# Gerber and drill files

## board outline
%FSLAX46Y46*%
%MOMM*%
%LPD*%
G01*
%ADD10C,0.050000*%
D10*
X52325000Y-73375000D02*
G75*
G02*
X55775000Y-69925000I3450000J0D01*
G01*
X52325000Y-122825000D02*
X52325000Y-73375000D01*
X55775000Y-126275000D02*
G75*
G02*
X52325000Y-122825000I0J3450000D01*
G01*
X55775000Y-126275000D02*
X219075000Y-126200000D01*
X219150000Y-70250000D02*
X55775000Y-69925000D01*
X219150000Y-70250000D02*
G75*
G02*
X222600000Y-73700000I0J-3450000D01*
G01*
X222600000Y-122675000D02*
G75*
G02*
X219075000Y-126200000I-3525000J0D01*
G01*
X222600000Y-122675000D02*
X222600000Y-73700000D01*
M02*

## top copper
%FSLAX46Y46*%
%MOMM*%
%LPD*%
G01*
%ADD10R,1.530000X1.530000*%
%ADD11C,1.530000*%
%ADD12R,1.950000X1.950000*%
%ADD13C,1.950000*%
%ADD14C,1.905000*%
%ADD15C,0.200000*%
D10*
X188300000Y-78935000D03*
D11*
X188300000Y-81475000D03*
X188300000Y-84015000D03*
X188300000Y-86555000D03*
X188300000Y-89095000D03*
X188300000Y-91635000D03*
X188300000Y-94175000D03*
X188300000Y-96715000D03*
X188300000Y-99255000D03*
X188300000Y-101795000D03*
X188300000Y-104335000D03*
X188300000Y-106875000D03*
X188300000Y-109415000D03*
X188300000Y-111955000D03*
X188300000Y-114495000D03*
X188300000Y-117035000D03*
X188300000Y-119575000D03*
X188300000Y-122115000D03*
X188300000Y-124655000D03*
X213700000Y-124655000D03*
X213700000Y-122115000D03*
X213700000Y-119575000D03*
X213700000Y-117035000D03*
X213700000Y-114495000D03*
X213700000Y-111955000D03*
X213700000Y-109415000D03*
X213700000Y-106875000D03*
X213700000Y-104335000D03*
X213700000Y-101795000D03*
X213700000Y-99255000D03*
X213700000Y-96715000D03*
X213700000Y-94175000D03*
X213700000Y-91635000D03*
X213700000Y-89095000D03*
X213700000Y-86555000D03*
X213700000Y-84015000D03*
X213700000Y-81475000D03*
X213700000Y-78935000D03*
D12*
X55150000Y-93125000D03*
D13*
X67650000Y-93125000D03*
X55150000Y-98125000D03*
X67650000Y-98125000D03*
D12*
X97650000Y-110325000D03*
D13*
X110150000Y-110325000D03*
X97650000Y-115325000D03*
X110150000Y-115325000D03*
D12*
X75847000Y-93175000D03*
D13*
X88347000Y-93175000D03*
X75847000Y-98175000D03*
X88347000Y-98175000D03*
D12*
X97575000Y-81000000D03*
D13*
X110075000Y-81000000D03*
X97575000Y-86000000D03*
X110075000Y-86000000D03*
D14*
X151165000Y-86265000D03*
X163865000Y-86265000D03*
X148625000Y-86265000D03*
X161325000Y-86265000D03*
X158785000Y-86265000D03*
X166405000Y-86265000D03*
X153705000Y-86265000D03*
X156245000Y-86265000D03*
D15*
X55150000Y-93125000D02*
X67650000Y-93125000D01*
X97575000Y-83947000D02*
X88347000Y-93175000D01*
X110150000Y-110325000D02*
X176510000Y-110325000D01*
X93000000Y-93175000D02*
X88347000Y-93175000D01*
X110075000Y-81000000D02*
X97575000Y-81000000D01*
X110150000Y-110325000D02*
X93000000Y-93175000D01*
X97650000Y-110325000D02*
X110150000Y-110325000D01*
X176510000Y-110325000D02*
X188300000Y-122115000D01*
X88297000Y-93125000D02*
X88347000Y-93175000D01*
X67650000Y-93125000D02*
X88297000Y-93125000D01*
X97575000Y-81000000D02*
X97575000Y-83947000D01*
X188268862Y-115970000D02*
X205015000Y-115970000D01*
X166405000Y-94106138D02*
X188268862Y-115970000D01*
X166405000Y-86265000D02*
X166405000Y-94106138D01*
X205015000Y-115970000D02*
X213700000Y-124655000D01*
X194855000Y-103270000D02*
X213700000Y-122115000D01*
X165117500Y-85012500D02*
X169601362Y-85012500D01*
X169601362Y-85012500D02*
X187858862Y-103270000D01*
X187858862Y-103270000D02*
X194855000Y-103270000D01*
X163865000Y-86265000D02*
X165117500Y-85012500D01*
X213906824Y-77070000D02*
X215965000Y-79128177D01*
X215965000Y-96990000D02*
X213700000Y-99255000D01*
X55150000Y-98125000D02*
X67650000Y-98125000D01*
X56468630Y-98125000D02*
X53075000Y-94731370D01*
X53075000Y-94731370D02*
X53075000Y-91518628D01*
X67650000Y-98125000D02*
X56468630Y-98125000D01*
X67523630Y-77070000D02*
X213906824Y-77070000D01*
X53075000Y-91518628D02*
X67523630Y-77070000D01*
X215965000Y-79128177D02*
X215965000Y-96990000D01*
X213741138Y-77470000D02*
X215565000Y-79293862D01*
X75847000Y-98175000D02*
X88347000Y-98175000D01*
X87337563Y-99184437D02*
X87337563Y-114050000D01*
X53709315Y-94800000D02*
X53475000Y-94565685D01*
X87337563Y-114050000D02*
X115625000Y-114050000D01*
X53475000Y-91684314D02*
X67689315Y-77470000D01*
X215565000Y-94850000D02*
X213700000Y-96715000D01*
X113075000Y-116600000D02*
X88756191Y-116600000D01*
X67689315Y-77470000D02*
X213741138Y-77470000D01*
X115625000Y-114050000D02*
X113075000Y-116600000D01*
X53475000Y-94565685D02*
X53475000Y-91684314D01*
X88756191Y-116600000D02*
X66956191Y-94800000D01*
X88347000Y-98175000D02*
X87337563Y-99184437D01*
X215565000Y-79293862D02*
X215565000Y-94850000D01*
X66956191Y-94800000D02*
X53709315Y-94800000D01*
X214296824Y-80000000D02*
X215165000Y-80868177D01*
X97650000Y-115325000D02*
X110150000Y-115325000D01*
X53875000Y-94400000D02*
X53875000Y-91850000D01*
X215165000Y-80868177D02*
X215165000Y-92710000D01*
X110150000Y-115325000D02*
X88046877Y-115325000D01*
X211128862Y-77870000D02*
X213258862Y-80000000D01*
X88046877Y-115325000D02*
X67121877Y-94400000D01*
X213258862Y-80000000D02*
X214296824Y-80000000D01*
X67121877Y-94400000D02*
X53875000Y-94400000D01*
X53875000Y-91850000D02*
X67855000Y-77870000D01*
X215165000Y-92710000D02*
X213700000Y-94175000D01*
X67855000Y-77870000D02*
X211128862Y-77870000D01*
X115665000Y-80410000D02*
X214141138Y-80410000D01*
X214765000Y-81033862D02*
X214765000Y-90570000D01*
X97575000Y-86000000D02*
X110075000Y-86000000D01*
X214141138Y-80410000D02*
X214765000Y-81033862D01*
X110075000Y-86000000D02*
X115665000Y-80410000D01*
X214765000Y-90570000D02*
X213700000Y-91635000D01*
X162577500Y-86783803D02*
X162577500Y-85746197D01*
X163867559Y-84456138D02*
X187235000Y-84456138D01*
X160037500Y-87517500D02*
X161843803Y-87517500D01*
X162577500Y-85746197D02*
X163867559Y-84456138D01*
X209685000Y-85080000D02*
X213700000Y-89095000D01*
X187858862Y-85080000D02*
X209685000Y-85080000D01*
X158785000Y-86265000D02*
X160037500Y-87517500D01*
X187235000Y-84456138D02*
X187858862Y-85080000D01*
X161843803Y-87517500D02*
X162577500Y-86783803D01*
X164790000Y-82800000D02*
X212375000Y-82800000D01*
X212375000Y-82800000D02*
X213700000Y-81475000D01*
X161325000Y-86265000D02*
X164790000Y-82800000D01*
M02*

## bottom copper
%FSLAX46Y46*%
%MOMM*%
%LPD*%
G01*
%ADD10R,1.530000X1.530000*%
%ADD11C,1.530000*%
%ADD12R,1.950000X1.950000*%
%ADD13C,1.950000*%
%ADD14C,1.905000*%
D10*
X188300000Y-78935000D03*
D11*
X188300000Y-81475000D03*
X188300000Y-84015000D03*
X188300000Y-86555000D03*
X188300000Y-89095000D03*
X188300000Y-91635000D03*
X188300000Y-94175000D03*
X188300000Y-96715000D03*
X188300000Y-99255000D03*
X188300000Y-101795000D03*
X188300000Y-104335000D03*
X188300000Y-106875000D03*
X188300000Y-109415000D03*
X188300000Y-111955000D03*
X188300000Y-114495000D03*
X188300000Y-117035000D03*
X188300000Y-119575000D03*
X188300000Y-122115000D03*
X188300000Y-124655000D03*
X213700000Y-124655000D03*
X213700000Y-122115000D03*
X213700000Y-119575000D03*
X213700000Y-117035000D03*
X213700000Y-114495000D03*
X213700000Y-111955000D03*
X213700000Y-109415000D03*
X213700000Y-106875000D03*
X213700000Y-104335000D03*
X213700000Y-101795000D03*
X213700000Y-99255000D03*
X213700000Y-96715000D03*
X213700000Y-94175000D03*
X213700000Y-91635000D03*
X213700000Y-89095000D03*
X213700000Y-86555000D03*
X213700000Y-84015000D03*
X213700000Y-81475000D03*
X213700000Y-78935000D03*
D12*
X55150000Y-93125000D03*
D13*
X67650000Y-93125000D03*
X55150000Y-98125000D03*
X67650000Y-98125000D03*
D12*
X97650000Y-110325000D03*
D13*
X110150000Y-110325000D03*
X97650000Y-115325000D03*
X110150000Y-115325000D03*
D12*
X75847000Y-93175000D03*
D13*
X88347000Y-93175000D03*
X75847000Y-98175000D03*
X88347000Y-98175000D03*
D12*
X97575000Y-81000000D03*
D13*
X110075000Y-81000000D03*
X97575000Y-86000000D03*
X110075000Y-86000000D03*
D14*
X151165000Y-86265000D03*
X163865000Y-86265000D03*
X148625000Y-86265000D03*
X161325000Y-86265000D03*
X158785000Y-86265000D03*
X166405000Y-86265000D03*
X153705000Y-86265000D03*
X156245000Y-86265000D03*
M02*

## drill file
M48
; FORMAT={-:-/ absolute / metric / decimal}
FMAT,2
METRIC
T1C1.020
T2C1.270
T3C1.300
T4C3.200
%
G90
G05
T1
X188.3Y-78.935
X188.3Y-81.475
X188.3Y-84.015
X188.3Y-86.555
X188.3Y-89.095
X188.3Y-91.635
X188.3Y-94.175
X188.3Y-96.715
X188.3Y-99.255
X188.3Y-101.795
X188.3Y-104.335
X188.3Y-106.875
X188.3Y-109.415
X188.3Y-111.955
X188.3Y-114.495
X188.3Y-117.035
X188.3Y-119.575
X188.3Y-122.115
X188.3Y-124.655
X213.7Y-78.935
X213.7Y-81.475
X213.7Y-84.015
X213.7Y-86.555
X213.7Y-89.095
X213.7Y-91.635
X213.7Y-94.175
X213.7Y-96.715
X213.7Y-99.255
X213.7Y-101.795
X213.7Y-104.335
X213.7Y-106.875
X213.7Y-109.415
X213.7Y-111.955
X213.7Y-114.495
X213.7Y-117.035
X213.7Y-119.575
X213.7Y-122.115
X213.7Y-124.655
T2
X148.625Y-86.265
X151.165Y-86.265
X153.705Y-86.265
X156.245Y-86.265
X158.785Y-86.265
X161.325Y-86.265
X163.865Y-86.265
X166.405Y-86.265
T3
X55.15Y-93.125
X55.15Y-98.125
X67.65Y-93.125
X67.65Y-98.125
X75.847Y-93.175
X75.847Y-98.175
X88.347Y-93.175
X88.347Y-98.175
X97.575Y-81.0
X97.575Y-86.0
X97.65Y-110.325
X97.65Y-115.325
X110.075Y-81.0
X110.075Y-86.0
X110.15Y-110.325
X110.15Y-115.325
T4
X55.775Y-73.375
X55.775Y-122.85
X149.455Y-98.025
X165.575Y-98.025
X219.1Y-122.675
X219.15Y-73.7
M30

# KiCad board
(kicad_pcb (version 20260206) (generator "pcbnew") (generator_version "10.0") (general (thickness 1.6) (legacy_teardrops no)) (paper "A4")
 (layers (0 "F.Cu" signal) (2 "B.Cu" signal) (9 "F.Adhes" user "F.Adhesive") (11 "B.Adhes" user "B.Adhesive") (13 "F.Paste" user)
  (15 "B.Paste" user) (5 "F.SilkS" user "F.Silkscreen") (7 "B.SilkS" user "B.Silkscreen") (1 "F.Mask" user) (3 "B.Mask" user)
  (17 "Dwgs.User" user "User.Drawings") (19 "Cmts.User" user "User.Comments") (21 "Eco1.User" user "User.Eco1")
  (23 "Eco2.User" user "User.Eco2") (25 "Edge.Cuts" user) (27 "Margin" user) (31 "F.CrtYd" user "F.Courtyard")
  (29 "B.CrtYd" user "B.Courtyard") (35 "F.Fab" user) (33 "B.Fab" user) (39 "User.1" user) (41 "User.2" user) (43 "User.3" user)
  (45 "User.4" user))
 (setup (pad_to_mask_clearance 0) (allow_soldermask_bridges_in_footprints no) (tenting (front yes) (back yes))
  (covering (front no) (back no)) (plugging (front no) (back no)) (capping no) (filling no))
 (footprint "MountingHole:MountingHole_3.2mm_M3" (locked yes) (layer "F.Cu") (at 55.775 122.85)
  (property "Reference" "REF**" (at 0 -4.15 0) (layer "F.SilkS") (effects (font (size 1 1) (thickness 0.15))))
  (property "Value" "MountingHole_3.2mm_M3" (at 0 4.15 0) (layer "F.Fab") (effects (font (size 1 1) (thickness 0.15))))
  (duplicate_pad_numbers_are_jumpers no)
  (pad "" np_thru_hole circle (at 0 0) (size 3.2 3.2) (drill 3.2) (layers "*.Cu" "*.Mask")))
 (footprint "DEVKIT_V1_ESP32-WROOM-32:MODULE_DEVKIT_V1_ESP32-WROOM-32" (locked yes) (layer "F.Cu") (at 201 101.785)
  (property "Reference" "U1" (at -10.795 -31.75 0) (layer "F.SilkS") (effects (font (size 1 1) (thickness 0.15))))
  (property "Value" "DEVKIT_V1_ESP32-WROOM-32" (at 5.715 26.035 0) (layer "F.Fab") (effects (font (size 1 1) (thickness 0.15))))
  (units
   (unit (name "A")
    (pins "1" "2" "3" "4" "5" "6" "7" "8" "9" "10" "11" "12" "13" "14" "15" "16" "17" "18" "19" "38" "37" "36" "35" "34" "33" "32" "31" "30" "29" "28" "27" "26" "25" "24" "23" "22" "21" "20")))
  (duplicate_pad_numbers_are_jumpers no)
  (pad "1" thru_hole rect (at -12.7 -22.85) (size 1.53 1.53) (drill 1.02) (layers "*.Cu" "*.Mask") (remove_unused_layers no)
   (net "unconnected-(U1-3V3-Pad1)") (solder_mask_margin 0.102))
  (pad "2" thru_hole circle (at -12.7 -20.31) (size 1.53 1.53) (drill 1.02) (layers "*.Cu" "*.Mask") (remove_unused_layers no)
   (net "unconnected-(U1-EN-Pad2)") (solder_mask_margin 0.102))
  (pad "3" thru_hole circle (at -12.7 -17.77) (size 1.53 1.53) (drill 1.02) (layers "*.Cu" "*.Mask") (remove_unused_layers no)
   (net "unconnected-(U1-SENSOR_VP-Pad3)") (solder_mask_margin 0.102))
  (pad "4" thru_hole circle (at -12.7 -15.23) (size 1.53 1.53) (drill 1.02) (layers "*.Cu" "*.Mask") (remove_unused_layers no)
   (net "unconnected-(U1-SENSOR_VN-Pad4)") (solder_mask_margin 0.102))
  (pad "5" thru_hole circle (at -12.7 -12.69) (size 1.53 1.53) (drill 1.02) (layers "*.Cu" "*.Mask") (remove_unused_layers no)
   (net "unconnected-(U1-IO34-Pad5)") (solder_mask_margin 0.102))
  (pad "6" thru_hole circle (at -12.7 -10.15) (size 1.53 1.53) (drill 1.02) (layers "*.Cu" "*.Mask") (remove_unused_layers no)
   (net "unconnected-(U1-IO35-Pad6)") (solder_mask_margin 0.102))
  (pad "7" thru_hole circle (at -12.7 -7.61) (size 1.53 1.53) (drill 1.02) (layers "*.Cu" "*.Mask") (remove_unused_layers no)
   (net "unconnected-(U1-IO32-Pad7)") (solder_mask_margin 0.102))
  (pad "8" thru_hole circle (at -12.7 -5.07) (size 1.53 1.53) (drill 1.02) (layers "*.Cu" "*.Mask") (remove_unused_layers no)
   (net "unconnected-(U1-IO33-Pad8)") (solder_mask_margin 0.102))
  (pad "9" thru_hole circle (at -12.7 -2.53) (size 1.53 1.53) (drill 1.02) (layers "*.Cu" "*.Mask") (remove_unused_layers no)
   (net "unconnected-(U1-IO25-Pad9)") (solder_mask_margin 0.102))
  (pad "10" thru_hole circle (at -12.7 0.01) (size 1.53 1.53) (drill 1.02) (layers "*.Cu" "*.Mask") (remove_unused_layers no)
   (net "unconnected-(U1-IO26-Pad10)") (solder_mask_margin 0.102))
  (pad "11" thru_hole circle (at -12.7 2.55) (size 1.53 1.53) (drill 1.02) (layers "*.Cu" "*.Mask") (remove_unused_layers no)
   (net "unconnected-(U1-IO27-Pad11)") (solder_mask_margin 0.102))
  (pad "12" thru_hole circle (at -12.7 5.09) (size 1.53 1.53) (drill 1.02) (layers "*.Cu" "*.Mask") (remove_unused_layers no)
   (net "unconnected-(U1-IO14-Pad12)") (solder_mask_margin 0.102))
  (pad "13" thru_hole circle (at -12.7 7.63) (size 1.53 1.53) (drill 1.02) (layers "*.Cu" "*.Mask") (remove_unused_layers no)
   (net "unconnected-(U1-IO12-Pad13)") (solder_mask_margin 0.102))
  (pad "14" thru_hole circle (at -12.7 10.17) (size 1.53 1.53) (drill 1.02) (layers "*.Cu" "*.Mask") (remove_unused_layers no)
   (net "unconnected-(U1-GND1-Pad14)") (solder_mask_margin 0.102))
  (pad "15" thru_hole circle (at -12.7 12.71) (size 1.53 1.53) (drill 1.02) (layers "*.Cu" "*.Mask") (remove_unused_layers no)
   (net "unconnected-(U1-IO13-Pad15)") (solder_mask_margin 0.102))
  (pad "16" thru_hole circle (at -12.7 15.25) (size 1.53 1.53) (drill 1.02) (layers "*.Cu" "*.Mask") (remove_unused_layers no)
   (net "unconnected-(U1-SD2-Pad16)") (solder_mask_margin 0.102))
  (pad "17" thru_hole circle (at -12.7 17.79) (size 1.53 1.53) (drill 1.02) (layers "*.Cu" "*.Mask") (remove_unused_layers no)
   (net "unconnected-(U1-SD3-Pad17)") (solder_mask_margin 0.102))
  (pad "18" thru_hole circle (at -12.7 20.33) (size 1.53 1.53) (drill 1.02) (layers "*.Cu" "*.Mask") (remove_unused_layers no)
   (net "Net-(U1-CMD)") (solder_mask_margin 0.102))
  (pad "19" thru_hole circle (at -12.7 22.87) (size 1.53 1.53) (drill 1.02) (layers "*.Cu" "*.Mask") (remove_unused_layers no)
   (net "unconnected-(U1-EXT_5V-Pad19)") (solder_mask_margin 0.102))
  (pad "20" thru_hole circle (at 12.7 22.87) (size 1.53 1.53) (drill 1.02) (layers "*.Cu" "*.Mask") (remove_unused_layers no)
   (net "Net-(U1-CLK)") (solder_mask_margin 0.102))
  (pad "21" thru_hole circle (at 12.7 20.33) (size 1.53 1.53) (drill 1.02) (layers "*.Cu" "*.Mask") (remove_unused_layers no)
   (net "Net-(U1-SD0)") (solder_mask_margin 0.102))
  (pad "22" thru_hole circle (at 12.7 17.79) (size 1.53 1.53) (drill 1.02) (layers "*.Cu" "*.Mask") (remove_unused_layers no)
   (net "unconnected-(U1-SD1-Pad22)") (solder_mask_margin 0.102))
  (pad "23" thru_hole circle (at 12.7 15.25) (size 1.53 1.53) (drill 1.02) (layers "*.Cu" "*.Mask") (remove_unused_layers no)
   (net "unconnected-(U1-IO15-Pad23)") (solder_mask_margin 0.102))
  (pad "24" thru_hole circle (at 12.7 12.71) (size 1.53 1.53) (drill 1.02) (layers "*.Cu" "*.Mask") (remove_unused_layers no)
   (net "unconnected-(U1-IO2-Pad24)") (solder_mask_margin 0.102))
  (pad "25" thru_hole circle (at 12.7 10.17) (size 1.53 1.53) (drill 1.02) (layers "*.Cu" "*.Mask") (remove_unused_layers no)
   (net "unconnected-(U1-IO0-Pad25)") (solder_mask_margin 0.102))
  (pad "26" thru_hole circle (at 12.7 7.63) (size 1.53 1.53) (drill 1.02) (layers "*.Cu" "*.Mask") (remove_unused_layers no)
   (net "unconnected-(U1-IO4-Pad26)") (solder_mask_margin 0.102))
  (pad "27" thru_hole circle (at 12.7 5.09) (size 1.53 1.53) (drill 1.02) (layers "*.Cu" "*.Mask") (remove_unused_layers no)
   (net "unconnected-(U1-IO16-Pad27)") (solder_mask_margin 0.102))
  (pad "28" thru_hole circle (at 12.7 2.55) (size 1.53 1.53) (drill 1.02) (layers "*.Cu" "*.Mask") (remove_unused_layers no)
   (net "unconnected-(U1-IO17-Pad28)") (solder_mask_margin 0.102))
  (pad "29" thru_hole circle (at 12.7 0.01) (size 1.53 1.53) (drill 1.02) (layers "*.Cu" "*.Mask") (remove_unused_layers no)
   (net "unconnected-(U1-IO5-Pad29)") (solder_mask_margin 0.102))
  (pad "30" thru_hole circle (at 12.7 -2.53) (size 1.53 1.53) (drill 1.02) (layers "*.Cu" "*.Mask") (remove_unused_layers no)
   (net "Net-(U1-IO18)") (solder_mask_margin 0.102))
  (pad "31" thru_hole circle (at 12.7 -5.07) (size 1.53 1.53) (drill 1.02) (layers "*.Cu" "*.Mask") (remove_unused_layers no)
   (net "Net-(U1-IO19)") (solder_mask_margin 0.102))
  (pad "32" thru_hole circle (at 12.7 -7.61) (size 1.53 1.53) (drill 1.02) (layers "*.Cu" "*.Mask") (remove_unused_layers no)
   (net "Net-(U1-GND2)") (solder_mask_margin 0.102))
  (pad "33" thru_hole circle (at 12.7 -10.15) (size 1.53 1.53) (drill 1.02) (layers "*.Cu" "*.Mask") (remove_unused_layers no)
   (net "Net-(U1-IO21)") (solder_mask_margin 0.102))
  (pad "34" thru_hole circle (at 12.7 -12.69) (size 1.53 1.53) (drill 1.02) (layers "*.Cu" "*.Mask") (remove_unused_layers no)
   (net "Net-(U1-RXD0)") (solder_mask_margin 0.102))
  (pad "35" thru_hole circle (at 12.7 -15.23) (size 1.53 1.53) (drill 1.02) (layers "*.Cu" "*.Mask") (remove_unused_layers no)
   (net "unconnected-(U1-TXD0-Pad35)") (solder_mask_margin 0.102))
  (pad "36" thru_hole circle (at 12.7 -17.77) (size 1.53 1.53) (drill 1.02) (layers "*.Cu" "*.Mask") (remove_unused_layers no)
   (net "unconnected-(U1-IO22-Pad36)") (solder_mask_margin 0.102))
  (pad "37" thru_hole circle (at 12.7 -20.31) (size 1.53 1.53) (drill 1.02) (layers "*.Cu" "*.Mask") (remove_unused_layers no)
   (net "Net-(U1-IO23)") (solder_mask_margin 0.102))
  (pad "38" thru_hole circle (at 12.7 -22.85) (size 1.53 1.53) (drill 1.02) (layers "*.Cu" "*.Mask") (remove_unused_layers no)
   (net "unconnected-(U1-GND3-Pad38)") (solder_mask_margin 0.102)))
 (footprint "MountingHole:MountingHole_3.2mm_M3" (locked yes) (layer "F.Cu") (at 55.775 73.375)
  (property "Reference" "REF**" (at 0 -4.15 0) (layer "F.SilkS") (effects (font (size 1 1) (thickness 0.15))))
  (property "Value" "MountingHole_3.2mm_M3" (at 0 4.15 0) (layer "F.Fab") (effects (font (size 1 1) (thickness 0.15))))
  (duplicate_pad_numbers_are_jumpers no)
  (pad "" np_thru_hole circle (at 0 0) (size 3.2 3.2) (drill 3.2) (layers "*.Cu" "*.Mask")))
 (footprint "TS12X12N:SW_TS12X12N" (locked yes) (layer "F.Cu") (at 61.4 95.625)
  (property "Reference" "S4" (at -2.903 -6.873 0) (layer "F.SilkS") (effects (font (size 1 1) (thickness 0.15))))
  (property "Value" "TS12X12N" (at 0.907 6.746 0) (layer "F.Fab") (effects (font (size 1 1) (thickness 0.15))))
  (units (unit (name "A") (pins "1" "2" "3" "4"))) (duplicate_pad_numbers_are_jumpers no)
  (pad "1" thru_hole rect (at -6.25 -2.5) (size 1.95 1.95) (drill 1.3) (layers "*.Cu" "*.Mask") (remove_unused_layers no)
   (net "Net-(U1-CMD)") (solder_mask_margin 0.102))
  (pad "2" thru_hole circle (at 6.25 -2.5) (size 1.95 1.95) (drill 1.3) (layers "*.Cu" "*.Mask") (remove_unused_layers no)
   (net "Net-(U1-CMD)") (solder_mask_margin 0.102))
  (pad "3" thru_hole circle (at -6.25 2.5) (size 1.95 1.95) (drill 1.3) (layers "*.Cu" "*.Mask") (remove_unused_layers no)
   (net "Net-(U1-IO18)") (solder_mask_margin 0.102))
  (pad "4" thru_hole circle (at 6.25 2.5) (size 1.95 1.95) (drill 1.3) (layers "*.Cu" "*.Mask") (remove_unused_layers no)
   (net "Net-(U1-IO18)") (solder_mask_margin 0.102)))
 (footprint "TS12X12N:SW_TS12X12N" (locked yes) (layer "F.Cu") (at 103.9 112.825)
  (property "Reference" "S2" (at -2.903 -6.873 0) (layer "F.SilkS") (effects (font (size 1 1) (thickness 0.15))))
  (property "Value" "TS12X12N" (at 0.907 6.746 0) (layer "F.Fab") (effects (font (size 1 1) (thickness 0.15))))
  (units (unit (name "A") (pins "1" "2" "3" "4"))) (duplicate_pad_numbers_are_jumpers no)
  (pad "1" thru_hole rect (at -6.25 -2.5) (size 1.95 1.95) (drill 1.3) (layers "*.Cu" "*.Mask") (remove_unused_layers no)
   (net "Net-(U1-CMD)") (solder_mask_margin 0.102))
  (pad "2" thru_hole circle (at 6.25 -2.5) (size 1.95 1.95) (drill 1.3) (layers "*.Cu" "*.Mask") (remove_unused_layers no)
   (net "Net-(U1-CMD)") (solder_mask_margin 0.102))
  (pad "3" thru_hole circle (at -6.25 2.5) (size 1.95 1.95) (drill 1.3) (layers "*.Cu" "*.Mask") (remove_unused_layers no)
   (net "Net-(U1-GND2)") (solder_mask_margin 0.102))
  (pad "4" thru_hole circle (at 6.25 2.5) (size 1.95 1.95) (drill 1.3) (layers "*.Cu" "*.Mask") (remove_unused_layers no)
   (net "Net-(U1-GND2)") (solder_mask_margin 0.102)))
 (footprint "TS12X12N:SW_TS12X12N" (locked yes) (layer "F.Cu") (at 82.097 95.675)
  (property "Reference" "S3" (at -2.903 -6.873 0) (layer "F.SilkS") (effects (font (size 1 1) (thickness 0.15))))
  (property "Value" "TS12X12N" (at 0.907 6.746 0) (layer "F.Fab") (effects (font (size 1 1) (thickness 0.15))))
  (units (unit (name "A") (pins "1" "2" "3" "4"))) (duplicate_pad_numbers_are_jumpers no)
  (pad "1" thru_hole rect (at -6.25 -2.5) (size 1.95 1.95) (drill 1.3) (layers "*.Cu" "*.Mask") (remove_unused_layers no)
   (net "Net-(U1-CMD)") (solder_mask_margin 0.102))
  (pad "2" thru_hole circle (at 6.25 -2.5) (size 1.95 1.95) (drill 1.3) (layers "*.Cu" "*.Mask") (remove_unused_layers no)
   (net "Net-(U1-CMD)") (solder_mask_margin 0.102))
  (pad "3" thru_hole circle (at -6.25 2.5) (size 1.95 1.95) (drill 1.3) (layers "*.Cu" "*.Mask") (remove_unused_layers no)
   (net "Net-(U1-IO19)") (solder_mask_margin 0.102))
  (pad "4" thru_hole circle (at 6.25 2.5) (size 1.95 1.95) (drill 1.3) (layers "*.Cu" "*.Mask") (remove_unused_layers no)
   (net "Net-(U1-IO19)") (solder_mask_margin 0.102)))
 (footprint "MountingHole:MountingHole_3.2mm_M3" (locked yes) (layer "F.Cu") (at 219.1 122.675)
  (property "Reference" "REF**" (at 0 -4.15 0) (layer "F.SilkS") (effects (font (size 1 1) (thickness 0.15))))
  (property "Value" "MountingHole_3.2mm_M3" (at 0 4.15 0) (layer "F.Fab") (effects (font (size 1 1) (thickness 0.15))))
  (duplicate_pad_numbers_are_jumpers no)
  (pad "" np_thru_hole circle (at 0 0) (size 3.2 3.2) (drill 3.2) (layers "*.Cu" "*.Mask")))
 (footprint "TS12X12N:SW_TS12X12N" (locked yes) (layer "F.Cu") (at 103.825 83.5)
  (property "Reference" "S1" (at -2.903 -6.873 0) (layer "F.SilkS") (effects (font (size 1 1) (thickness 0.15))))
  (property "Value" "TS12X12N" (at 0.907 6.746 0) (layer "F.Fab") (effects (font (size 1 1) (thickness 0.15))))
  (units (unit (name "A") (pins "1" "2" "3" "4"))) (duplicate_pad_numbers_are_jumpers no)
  (pad "1" thru_hole rect (at -6.25 -2.5) (size 1.95 1.95) (drill 1.3) (layers "*.Cu" "*.Mask") (remove_unused_layers no)
   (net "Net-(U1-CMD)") (solder_mask_margin 0.102))
  (pad "2" thru_hole circle (at 6.25 -2.5) (size 1.95 1.95) (drill 1.3) (layers "*.Cu" "*.Mask") (remove_unused_layers no)
   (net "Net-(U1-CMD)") (solder_mask_margin 0.102))
  (pad "3" thru_hole circle (at -6.25 2.5) (size 1.95 1.95) (drill 1.3) (layers "*.Cu" "*.Mask") (remove_unused_layers no)
   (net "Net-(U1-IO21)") (solder_mask_margin 0.102))
  (pad "4" thru_hole circle (at 6.25 2.5) (size 1.95 1.95) (drill 1.3) (layers "*.Cu" "*.Mask") (remove_unused_layers no)
   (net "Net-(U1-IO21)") (solder_mask_margin 0.102)))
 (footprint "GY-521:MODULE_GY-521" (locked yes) (layer "F.Cu") (at 157.515 92.595 -90)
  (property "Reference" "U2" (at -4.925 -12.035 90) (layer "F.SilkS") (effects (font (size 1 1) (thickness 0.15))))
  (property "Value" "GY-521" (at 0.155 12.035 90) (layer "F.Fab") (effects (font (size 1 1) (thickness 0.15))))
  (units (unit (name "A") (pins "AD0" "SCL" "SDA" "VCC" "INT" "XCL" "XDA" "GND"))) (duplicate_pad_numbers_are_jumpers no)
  (pad "" np_thru_hole circle (at 5.43 -8.06 270) (size 3.2 3.2) (drill 3.2) (layers "*.Cu" "*.Mask"))
  (pad "" np_thru_hole circle (at 5.43 8.06 270) (size 3.2 3.2) (drill 3.2) (layers "*.Cu" "*.Mask"))
  (pad "AD0" thru_hole circle (at -6.33 6.35 270) (size 1.905 1.905) (drill 1.27) (layers "*.Cu" "*.Mask") (remove_unused_layers no)
   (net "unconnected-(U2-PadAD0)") (solder_mask_margin 0.102))
  (pad "GND" thru_hole circle (at -6.33 -6.35 270) (size 1.905 1.905) (drill 1.27) (layers "*.Cu" "*.Mask") (remove_unused_layers no)
   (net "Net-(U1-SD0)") (solder_mask_margin 0.102))
  (pad "INT" thru_hole circle (at -6.33 8.89 270) (size 1.905 1.905) (drill 1.27) (layers "*.Cu" "*.Mask") (remove_unused_layers no)
   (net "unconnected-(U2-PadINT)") (solder_mask_margin 0.102))
  (pad "SCL" thru_hole circle (at -6.33 -3.81 270) (size 1.905 1.905) (drill 1.27) (layers "*.Cu" "*.Mask") (remove_unused_layers no)
   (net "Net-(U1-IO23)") (solder_mask_margin 0.102))
  (pad "SDA" thru_hole circle (at -6.33 -1.27 270) (size 1.905 1.905) (drill 1.27) (layers "*.Cu" "*.Mask") (remove_unused_layers no)
   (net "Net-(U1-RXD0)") (solder_mask_margin 0.102))
  (pad "VCC" thru_hole circle (at -6.33 -8.89 270) (size 1.905 1.905) (drill 1.27) (layers "*.Cu" "*.Mask") (remove_unused_layers no)
   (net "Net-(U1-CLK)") (solder_mask_margin 0.102))
  (pad "XCL" thru_hole circle (at -6.33 3.81 270) (size 1.905 1.905) (drill 1.27) (layers "*.Cu" "*.Mask") (remove_unused_layers no)
   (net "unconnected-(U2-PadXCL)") (solder_mask_margin 0.102))
  (pad "XDA" thru_hole circle (at -6.33 1.27 270) (size 1.905 1.905) (drill 1.27) (layers "*.Cu" "*.Mask") (remove_unused_layers no)
   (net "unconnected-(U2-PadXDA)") (solder_mask_margin 0.102)))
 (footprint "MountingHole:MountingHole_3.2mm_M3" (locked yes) (layer "F.Cu") (at 219.15 73.7)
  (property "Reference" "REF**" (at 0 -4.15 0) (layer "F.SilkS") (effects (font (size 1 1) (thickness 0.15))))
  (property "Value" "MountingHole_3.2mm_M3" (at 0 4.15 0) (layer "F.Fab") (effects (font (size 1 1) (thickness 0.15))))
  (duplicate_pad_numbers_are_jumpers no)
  (pad "" np_thru_hole circle (at 0 0) (size 3.2 3.2) (drill 3.2) (layers "*.Cu" "*.Mask")))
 (gr_arc (start 52.325 73.375) (mid 53.335482 70.935482) (end 55.775 69.925) (stroke (width 0.05) (type default)) (locked yes)
  (layer "Edge.Cuts"))
 (gr_line (start 52.325 122.825) (end 52.325 73.375) (stroke (width 0.05) (type default)) (locked yes) (layer "Edge.Cuts"))
 (gr_arc (start 55.775 126.275) (mid 53.335482 125.264518) (end 52.325 122.825) (stroke (width 0.05) (type default)) (locked yes)
  (layer "Edge.Cuts"))
 (gr_line (start 55.775 126.275) (end 219.075 126.2) (stroke (width 0.05) (type default)) (locked yes) (layer "Edge.Cuts"))
 (gr_line (start 219.15 70.25) (end 55.775 69.925) (stroke (width 0.05) (type default)) (locked yes) (layer "Edge.Cuts"))
 (gr_arc (start 219.15 70.25) (mid 221.589518 71.260482) (end 222.6 73.7) (stroke (width 0.05) (type default)) (locked yes)
  (layer "Edge.Cuts"))
 (gr_arc (start 222.6 122.675) (mid 221.567551 125.167551) (end 219.075 126.2) (stroke (width 0.05) (type default)) (locked yes)
  (layer "Edge.Cuts"))
 (gr_line (start 222.6 122.675) (end 222.6 73.7) (stroke (width 0.05) (type default)) (locked yes) (layer "Edge.Cuts"))
 (segment (start 55.15 93.125) (end 67.65 93.125) (width 0.2) (locked yes) (layer "F.Cu") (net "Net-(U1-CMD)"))
 (segment (start 97.575 83.947) (end 88.347 93.175) (width 0.2) (locked yes) (layer "F.Cu") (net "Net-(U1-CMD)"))
 (segment (start 110.15 110.325) (end 176.51 110.325) (width 0.2) (locked yes) (layer "F.Cu") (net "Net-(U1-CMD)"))
 (segment (start 93 93.175) (end 88.347 93.175) (width 0.2) (locked yes) (layer "F.Cu") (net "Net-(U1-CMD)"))
 (segment (start 110.075 81) (end 97.575 81) (width 0.2) (locked yes) (layer "F.Cu") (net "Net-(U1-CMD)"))
 (segment (start 110.15 110.325) (end 93 93.175) (width 0.2) (locked yes) (layer "F.Cu") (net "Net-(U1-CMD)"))
 (segment (start 97.65 110.325) (end 110.15 110.325) (width 0.2) (locked yes) (layer "F.Cu") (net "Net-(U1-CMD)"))
 (segment (start 176.51 110.325) (end 188.3 122.115) (width 0.2) (locked yes) (layer "F.Cu") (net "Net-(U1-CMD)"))
 (segment (start 88.297 93.125) (end 88.347 93.175) (width 0.2) (locked yes) (layer "F.Cu") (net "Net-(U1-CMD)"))
 (segment (start 67.65 93.125) (end 88.297 93.125) (width 0.2) (locked yes) (layer "F.Cu") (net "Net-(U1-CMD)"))
 (segment (start 97.575 81) (end 97.575 83.947) (width 0.2) (locked yes) (layer "F.Cu") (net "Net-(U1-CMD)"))
 (segment (start 188.268862 115.97) (end 205.015 115.97) (width 0.2) (locked yes) (layer "F.Cu") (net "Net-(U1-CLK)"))
 (segment (start 166.405 94.106138) (end 188.268862 115.97) (width 0.2) (locked yes) (layer "F.Cu") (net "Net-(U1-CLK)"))
 (segment (start 166.405 86.265) (end 166.405 94.106138) (width 0.2) (locked yes) (layer "F.Cu") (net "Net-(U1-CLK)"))
 (segment (start 205.015 115.97) (end 213.7 124.655) (width 0.2) (locked yes) (layer "F.Cu") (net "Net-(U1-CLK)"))
 (segment (start 194.855 103.27) (end 213.7 122.115) (width 0.2) (locked yes) (layer "F.Cu") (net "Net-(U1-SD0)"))
 (segment (start 165.1175 85.0125) (end 169.601362 85.0125) (width 0.2) (locked yes) (layer "F.Cu") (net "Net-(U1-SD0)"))
 (segment (start 169.601362 85.0125) (end 187.858862 103.27) (width 0.2) (locked yes) (layer "F.Cu") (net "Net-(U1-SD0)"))
 (segment (start 187.858862 103.27) (end 194.855 103.27) (width 0.2) (locked yes) (layer "F.Cu") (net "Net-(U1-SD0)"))
 (segment (start 163.865 86.265) (end 165.1175 85.0125) (width 0.2) (locked yes) (layer "F.Cu") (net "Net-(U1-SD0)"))
 (segment (start 213.906824 77.07) (end 215.965 79.128177) (width 0.2) (locked yes) (layer "F.Cu") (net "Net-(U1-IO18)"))
 (segment (start 215.965 96.99) (end 213.7 99.255) (width 0.2) (locked yes) (layer "F.Cu") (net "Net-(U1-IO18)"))
 (segment (start 55.15 98.125) (end 67.65 98.125) (width 0.2) (locked yes) (layer "F.Cu") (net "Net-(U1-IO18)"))
 (segment (start 56.46863 98.125) (end 53.075 94.73137) (width 0.2) (locked yes) (layer "F.Cu") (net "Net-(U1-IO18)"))
 (segment (start 53.075 94.73137) (end 53.075 91.518628) (width 0.2) (locked yes) (layer "F.Cu") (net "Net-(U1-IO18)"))
 (segment (start 67.65 98.125) (end 56.46863 98.125) (width 0.2) (locked yes) (layer "F.Cu") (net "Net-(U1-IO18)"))
 (segment (start 67.52363 77.07) (end 213.906824 77.07) (width 0.2) (locked yes) (layer "F.Cu") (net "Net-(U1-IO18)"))
 (segment (start 53.075 91.518628) (end 67.52363 77.07) (width 0.2) (locked yes) (layer "F.Cu") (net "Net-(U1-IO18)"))
 (segment (start 215.965 79.128177) (end 215.965 96.99) (width 0.2) (locked yes) (layer "F.Cu") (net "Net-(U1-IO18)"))
 (segment (start 213.741138 77.47) (end 215.565 79.293862) (width 0.2) (locked yes) (layer "F.Cu") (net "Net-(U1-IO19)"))
 (segment (start 75.847 98.175) (end 88.347 98.175) (width 0.2) (locked yes) (layer "F.Cu") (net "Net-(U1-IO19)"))
 (segment (start 87.337563 99.184437) (end 87.337563 114.05) (width 0.2) (locked yes) (layer "F.Cu") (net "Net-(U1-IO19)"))
 (segment (start 53.709315 94.8) (end 53.475 94.565685) (width 0.2) (locked yes) (layer "F.Cu") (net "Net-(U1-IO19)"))
 (segment (start 87.337563 114.05) (end 115.625 114.05) (width 0.2) (locked yes) (layer "F.Cu") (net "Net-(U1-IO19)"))
 (segment (start 53.475 91.684314) (end 67.689315 77.47) (width 0.2) (locked yes) (layer "F.Cu") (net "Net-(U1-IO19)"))
 (segment (start 215.565 94.85) (end 213.7 96.715) (width 0.2) (locked yes) (layer "F.Cu") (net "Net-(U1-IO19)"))
 (segment (start 113.075 116.6) (end 88.756191 116.6) (width 0.2) (locked yes) (layer "F.Cu") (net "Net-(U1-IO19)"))
 (segment (start 67.689315 77.47) (end 213.741138 77.47) (width 0.2) (locked yes) (layer "F.Cu") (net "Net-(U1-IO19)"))
 (segment (start 115.625 114.05) (end 113.075 116.6) (width 0.2) (locked yes) (layer "F.Cu") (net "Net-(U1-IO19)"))
 (segment (start 53.475 94.565685) (end 53.475 91.684314) (width 0.2) (locked yes) (layer "F.Cu") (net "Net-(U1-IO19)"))
 (segment (start 88.756191 116.6) (end 66.956191 94.8) (width 0.2) (locked yes) (layer "F.Cu") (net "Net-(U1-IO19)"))
 (segment (start 88.347 98.175) (end 87.337563 99.184437) (width 0.2) (locked yes) (layer "F.Cu") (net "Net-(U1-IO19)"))
 (segment (start 215.565 79.293862) (end 215.565 94.85) (width 0.2) (locked yes) (layer "F.Cu") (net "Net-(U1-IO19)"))
 (segment (start 66.956191 94.8) (end 53.709315 94.8) (width 0.2) (locked yes) (layer "F.Cu") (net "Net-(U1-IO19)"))
 (segment (start 214.296824 80) (end 215.165 80.868177) (width 0.2) (locked yes) (layer "F.Cu") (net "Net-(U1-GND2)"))
 (segment (start 97.65 115.325) (end 110.15 115.325) (width 0.2) (locked yes) (layer "F.Cu") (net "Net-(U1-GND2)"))
 (segment (start 53.875 94.4) (end 53.875 91.85) (width 0.2) (locked yes) (layer "F.Cu") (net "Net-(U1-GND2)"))
 (segment (start 215.165 80.868177) (end 215.165 92.71) (width 0.2) (locked yes) (layer "F.Cu") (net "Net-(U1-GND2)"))
 (segment (start 110.15 115.325) (end 88.046877 115.325) (width 0.2) (locked yes) (layer "F.Cu") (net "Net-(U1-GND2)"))
 (segment (start 211.128862 77.87) (end 213.258862 80) (width 0.2) (locked yes) (layer "F.Cu") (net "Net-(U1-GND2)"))
 (segment (start 88.046877 115.325) (end 67.121877 94.4) (width 0.2) (locked yes) (layer "F.Cu") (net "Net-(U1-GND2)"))
 (segment (start 213.258862 80) (end 214.296824 80) (width 0.2) (locked yes) (layer "F.Cu") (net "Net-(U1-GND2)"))
 (segment (start 67.121877 94.4) (end 53.875 94.4) (width 0.2) (locked yes) (layer "F.Cu") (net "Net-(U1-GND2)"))
 (segment (start 53.875 91.85) (end 67.855 77.87) (width 0.2) (locked yes) (layer "F.Cu") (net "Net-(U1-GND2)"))
 (segment (start 215.165 92.71) (end 213.7 94.175) (width 0.2) (locked yes) (layer "F.Cu") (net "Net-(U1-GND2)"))
 (segment (start 67.855 77.87) (end 211.128862 77.87) (width 0.2) (locked yes) (layer "F.Cu") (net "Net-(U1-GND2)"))
 (segment (start 115.665 80.41) (end 214.141138 80.41) (width 0.2) (locked yes) (layer "F.Cu") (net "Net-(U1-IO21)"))
 (segment (start 214.765 81.033862) (end 214.765 90.57) (width 0.2) (locked yes) (layer "F.Cu") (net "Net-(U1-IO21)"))
 (segment (start 97.575 86) (end 110.075 86) (width 0.2) (locked yes) (layer "F.Cu") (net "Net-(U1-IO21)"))
 (segment (start 214.141138 80.41) (end 214.765 81.033862) (width 0.2) (locked yes) (layer "F.Cu") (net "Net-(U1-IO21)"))
 (segment (start 110.075 86) (end 115.665 80.41) (width 0.2) (locked yes) (layer "F.Cu") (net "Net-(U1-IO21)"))
 (segment (start 214.765 90.57) (end 213.7 91.635) (width 0.2) (locked yes) (layer "F.Cu") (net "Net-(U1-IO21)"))
 (segment (start 162.5775 86.783803) (end 162.5775 85.746197) (width 0.2) (locked yes) (layer "F.Cu") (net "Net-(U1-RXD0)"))
 (segment (start 163.867559 84.456138) (end 187.235 84.456138) (width 0.2) (locked yes) (layer "F.Cu") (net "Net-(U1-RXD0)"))
 (segment (start 160.0375 87.5175) (end 161.843803 87.5175) (width 0.2) (locked yes) (layer "F.Cu") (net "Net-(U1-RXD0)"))
 (segment (start 162.5775 85.746197) (end 163.867559 84.456138) (width 0.2) (locked yes) (layer "F.Cu") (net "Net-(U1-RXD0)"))
 (segment (start 209.685 85.08) (end 213.7 89.095) (width 0.2) (locked yes) (layer "F.Cu") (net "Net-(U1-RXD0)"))
 (segment (start 187.858862 85.08) (end 209.685 85.08) (width 0.2) (locked yes) (layer "F.Cu") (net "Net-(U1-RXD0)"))
 (segment (start 158.785 86.265) (end 160.0375 87.5175) (width 0.2) (locked yes) (layer "F.Cu") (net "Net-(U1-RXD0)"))
 (segment (start 187.235 84.456138) (end 187.858862 85.08) (width 0.2) (locked yes) (layer "F.Cu") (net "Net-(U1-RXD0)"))
 (segment (start 161.843803 87.5175) (end 162.5775 86.783803) (width 0.2) (locked yes) (layer "F.Cu") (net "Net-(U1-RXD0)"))
 (segment (start 164.79 82.8) (end 212.375 82.8) (width 0.2) (locked yes) (layer "F.Cu") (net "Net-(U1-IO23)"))
 (segment (start 212.375 82.8) (end 213.7 81.475) (width 0.2) (locked yes) (layer "F.Cu") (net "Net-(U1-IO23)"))
 (segment (start 161.325 86.265) (end 164.79 82.8) (width 0.2) (locked yes) (layer "F.Cu") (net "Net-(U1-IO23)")))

